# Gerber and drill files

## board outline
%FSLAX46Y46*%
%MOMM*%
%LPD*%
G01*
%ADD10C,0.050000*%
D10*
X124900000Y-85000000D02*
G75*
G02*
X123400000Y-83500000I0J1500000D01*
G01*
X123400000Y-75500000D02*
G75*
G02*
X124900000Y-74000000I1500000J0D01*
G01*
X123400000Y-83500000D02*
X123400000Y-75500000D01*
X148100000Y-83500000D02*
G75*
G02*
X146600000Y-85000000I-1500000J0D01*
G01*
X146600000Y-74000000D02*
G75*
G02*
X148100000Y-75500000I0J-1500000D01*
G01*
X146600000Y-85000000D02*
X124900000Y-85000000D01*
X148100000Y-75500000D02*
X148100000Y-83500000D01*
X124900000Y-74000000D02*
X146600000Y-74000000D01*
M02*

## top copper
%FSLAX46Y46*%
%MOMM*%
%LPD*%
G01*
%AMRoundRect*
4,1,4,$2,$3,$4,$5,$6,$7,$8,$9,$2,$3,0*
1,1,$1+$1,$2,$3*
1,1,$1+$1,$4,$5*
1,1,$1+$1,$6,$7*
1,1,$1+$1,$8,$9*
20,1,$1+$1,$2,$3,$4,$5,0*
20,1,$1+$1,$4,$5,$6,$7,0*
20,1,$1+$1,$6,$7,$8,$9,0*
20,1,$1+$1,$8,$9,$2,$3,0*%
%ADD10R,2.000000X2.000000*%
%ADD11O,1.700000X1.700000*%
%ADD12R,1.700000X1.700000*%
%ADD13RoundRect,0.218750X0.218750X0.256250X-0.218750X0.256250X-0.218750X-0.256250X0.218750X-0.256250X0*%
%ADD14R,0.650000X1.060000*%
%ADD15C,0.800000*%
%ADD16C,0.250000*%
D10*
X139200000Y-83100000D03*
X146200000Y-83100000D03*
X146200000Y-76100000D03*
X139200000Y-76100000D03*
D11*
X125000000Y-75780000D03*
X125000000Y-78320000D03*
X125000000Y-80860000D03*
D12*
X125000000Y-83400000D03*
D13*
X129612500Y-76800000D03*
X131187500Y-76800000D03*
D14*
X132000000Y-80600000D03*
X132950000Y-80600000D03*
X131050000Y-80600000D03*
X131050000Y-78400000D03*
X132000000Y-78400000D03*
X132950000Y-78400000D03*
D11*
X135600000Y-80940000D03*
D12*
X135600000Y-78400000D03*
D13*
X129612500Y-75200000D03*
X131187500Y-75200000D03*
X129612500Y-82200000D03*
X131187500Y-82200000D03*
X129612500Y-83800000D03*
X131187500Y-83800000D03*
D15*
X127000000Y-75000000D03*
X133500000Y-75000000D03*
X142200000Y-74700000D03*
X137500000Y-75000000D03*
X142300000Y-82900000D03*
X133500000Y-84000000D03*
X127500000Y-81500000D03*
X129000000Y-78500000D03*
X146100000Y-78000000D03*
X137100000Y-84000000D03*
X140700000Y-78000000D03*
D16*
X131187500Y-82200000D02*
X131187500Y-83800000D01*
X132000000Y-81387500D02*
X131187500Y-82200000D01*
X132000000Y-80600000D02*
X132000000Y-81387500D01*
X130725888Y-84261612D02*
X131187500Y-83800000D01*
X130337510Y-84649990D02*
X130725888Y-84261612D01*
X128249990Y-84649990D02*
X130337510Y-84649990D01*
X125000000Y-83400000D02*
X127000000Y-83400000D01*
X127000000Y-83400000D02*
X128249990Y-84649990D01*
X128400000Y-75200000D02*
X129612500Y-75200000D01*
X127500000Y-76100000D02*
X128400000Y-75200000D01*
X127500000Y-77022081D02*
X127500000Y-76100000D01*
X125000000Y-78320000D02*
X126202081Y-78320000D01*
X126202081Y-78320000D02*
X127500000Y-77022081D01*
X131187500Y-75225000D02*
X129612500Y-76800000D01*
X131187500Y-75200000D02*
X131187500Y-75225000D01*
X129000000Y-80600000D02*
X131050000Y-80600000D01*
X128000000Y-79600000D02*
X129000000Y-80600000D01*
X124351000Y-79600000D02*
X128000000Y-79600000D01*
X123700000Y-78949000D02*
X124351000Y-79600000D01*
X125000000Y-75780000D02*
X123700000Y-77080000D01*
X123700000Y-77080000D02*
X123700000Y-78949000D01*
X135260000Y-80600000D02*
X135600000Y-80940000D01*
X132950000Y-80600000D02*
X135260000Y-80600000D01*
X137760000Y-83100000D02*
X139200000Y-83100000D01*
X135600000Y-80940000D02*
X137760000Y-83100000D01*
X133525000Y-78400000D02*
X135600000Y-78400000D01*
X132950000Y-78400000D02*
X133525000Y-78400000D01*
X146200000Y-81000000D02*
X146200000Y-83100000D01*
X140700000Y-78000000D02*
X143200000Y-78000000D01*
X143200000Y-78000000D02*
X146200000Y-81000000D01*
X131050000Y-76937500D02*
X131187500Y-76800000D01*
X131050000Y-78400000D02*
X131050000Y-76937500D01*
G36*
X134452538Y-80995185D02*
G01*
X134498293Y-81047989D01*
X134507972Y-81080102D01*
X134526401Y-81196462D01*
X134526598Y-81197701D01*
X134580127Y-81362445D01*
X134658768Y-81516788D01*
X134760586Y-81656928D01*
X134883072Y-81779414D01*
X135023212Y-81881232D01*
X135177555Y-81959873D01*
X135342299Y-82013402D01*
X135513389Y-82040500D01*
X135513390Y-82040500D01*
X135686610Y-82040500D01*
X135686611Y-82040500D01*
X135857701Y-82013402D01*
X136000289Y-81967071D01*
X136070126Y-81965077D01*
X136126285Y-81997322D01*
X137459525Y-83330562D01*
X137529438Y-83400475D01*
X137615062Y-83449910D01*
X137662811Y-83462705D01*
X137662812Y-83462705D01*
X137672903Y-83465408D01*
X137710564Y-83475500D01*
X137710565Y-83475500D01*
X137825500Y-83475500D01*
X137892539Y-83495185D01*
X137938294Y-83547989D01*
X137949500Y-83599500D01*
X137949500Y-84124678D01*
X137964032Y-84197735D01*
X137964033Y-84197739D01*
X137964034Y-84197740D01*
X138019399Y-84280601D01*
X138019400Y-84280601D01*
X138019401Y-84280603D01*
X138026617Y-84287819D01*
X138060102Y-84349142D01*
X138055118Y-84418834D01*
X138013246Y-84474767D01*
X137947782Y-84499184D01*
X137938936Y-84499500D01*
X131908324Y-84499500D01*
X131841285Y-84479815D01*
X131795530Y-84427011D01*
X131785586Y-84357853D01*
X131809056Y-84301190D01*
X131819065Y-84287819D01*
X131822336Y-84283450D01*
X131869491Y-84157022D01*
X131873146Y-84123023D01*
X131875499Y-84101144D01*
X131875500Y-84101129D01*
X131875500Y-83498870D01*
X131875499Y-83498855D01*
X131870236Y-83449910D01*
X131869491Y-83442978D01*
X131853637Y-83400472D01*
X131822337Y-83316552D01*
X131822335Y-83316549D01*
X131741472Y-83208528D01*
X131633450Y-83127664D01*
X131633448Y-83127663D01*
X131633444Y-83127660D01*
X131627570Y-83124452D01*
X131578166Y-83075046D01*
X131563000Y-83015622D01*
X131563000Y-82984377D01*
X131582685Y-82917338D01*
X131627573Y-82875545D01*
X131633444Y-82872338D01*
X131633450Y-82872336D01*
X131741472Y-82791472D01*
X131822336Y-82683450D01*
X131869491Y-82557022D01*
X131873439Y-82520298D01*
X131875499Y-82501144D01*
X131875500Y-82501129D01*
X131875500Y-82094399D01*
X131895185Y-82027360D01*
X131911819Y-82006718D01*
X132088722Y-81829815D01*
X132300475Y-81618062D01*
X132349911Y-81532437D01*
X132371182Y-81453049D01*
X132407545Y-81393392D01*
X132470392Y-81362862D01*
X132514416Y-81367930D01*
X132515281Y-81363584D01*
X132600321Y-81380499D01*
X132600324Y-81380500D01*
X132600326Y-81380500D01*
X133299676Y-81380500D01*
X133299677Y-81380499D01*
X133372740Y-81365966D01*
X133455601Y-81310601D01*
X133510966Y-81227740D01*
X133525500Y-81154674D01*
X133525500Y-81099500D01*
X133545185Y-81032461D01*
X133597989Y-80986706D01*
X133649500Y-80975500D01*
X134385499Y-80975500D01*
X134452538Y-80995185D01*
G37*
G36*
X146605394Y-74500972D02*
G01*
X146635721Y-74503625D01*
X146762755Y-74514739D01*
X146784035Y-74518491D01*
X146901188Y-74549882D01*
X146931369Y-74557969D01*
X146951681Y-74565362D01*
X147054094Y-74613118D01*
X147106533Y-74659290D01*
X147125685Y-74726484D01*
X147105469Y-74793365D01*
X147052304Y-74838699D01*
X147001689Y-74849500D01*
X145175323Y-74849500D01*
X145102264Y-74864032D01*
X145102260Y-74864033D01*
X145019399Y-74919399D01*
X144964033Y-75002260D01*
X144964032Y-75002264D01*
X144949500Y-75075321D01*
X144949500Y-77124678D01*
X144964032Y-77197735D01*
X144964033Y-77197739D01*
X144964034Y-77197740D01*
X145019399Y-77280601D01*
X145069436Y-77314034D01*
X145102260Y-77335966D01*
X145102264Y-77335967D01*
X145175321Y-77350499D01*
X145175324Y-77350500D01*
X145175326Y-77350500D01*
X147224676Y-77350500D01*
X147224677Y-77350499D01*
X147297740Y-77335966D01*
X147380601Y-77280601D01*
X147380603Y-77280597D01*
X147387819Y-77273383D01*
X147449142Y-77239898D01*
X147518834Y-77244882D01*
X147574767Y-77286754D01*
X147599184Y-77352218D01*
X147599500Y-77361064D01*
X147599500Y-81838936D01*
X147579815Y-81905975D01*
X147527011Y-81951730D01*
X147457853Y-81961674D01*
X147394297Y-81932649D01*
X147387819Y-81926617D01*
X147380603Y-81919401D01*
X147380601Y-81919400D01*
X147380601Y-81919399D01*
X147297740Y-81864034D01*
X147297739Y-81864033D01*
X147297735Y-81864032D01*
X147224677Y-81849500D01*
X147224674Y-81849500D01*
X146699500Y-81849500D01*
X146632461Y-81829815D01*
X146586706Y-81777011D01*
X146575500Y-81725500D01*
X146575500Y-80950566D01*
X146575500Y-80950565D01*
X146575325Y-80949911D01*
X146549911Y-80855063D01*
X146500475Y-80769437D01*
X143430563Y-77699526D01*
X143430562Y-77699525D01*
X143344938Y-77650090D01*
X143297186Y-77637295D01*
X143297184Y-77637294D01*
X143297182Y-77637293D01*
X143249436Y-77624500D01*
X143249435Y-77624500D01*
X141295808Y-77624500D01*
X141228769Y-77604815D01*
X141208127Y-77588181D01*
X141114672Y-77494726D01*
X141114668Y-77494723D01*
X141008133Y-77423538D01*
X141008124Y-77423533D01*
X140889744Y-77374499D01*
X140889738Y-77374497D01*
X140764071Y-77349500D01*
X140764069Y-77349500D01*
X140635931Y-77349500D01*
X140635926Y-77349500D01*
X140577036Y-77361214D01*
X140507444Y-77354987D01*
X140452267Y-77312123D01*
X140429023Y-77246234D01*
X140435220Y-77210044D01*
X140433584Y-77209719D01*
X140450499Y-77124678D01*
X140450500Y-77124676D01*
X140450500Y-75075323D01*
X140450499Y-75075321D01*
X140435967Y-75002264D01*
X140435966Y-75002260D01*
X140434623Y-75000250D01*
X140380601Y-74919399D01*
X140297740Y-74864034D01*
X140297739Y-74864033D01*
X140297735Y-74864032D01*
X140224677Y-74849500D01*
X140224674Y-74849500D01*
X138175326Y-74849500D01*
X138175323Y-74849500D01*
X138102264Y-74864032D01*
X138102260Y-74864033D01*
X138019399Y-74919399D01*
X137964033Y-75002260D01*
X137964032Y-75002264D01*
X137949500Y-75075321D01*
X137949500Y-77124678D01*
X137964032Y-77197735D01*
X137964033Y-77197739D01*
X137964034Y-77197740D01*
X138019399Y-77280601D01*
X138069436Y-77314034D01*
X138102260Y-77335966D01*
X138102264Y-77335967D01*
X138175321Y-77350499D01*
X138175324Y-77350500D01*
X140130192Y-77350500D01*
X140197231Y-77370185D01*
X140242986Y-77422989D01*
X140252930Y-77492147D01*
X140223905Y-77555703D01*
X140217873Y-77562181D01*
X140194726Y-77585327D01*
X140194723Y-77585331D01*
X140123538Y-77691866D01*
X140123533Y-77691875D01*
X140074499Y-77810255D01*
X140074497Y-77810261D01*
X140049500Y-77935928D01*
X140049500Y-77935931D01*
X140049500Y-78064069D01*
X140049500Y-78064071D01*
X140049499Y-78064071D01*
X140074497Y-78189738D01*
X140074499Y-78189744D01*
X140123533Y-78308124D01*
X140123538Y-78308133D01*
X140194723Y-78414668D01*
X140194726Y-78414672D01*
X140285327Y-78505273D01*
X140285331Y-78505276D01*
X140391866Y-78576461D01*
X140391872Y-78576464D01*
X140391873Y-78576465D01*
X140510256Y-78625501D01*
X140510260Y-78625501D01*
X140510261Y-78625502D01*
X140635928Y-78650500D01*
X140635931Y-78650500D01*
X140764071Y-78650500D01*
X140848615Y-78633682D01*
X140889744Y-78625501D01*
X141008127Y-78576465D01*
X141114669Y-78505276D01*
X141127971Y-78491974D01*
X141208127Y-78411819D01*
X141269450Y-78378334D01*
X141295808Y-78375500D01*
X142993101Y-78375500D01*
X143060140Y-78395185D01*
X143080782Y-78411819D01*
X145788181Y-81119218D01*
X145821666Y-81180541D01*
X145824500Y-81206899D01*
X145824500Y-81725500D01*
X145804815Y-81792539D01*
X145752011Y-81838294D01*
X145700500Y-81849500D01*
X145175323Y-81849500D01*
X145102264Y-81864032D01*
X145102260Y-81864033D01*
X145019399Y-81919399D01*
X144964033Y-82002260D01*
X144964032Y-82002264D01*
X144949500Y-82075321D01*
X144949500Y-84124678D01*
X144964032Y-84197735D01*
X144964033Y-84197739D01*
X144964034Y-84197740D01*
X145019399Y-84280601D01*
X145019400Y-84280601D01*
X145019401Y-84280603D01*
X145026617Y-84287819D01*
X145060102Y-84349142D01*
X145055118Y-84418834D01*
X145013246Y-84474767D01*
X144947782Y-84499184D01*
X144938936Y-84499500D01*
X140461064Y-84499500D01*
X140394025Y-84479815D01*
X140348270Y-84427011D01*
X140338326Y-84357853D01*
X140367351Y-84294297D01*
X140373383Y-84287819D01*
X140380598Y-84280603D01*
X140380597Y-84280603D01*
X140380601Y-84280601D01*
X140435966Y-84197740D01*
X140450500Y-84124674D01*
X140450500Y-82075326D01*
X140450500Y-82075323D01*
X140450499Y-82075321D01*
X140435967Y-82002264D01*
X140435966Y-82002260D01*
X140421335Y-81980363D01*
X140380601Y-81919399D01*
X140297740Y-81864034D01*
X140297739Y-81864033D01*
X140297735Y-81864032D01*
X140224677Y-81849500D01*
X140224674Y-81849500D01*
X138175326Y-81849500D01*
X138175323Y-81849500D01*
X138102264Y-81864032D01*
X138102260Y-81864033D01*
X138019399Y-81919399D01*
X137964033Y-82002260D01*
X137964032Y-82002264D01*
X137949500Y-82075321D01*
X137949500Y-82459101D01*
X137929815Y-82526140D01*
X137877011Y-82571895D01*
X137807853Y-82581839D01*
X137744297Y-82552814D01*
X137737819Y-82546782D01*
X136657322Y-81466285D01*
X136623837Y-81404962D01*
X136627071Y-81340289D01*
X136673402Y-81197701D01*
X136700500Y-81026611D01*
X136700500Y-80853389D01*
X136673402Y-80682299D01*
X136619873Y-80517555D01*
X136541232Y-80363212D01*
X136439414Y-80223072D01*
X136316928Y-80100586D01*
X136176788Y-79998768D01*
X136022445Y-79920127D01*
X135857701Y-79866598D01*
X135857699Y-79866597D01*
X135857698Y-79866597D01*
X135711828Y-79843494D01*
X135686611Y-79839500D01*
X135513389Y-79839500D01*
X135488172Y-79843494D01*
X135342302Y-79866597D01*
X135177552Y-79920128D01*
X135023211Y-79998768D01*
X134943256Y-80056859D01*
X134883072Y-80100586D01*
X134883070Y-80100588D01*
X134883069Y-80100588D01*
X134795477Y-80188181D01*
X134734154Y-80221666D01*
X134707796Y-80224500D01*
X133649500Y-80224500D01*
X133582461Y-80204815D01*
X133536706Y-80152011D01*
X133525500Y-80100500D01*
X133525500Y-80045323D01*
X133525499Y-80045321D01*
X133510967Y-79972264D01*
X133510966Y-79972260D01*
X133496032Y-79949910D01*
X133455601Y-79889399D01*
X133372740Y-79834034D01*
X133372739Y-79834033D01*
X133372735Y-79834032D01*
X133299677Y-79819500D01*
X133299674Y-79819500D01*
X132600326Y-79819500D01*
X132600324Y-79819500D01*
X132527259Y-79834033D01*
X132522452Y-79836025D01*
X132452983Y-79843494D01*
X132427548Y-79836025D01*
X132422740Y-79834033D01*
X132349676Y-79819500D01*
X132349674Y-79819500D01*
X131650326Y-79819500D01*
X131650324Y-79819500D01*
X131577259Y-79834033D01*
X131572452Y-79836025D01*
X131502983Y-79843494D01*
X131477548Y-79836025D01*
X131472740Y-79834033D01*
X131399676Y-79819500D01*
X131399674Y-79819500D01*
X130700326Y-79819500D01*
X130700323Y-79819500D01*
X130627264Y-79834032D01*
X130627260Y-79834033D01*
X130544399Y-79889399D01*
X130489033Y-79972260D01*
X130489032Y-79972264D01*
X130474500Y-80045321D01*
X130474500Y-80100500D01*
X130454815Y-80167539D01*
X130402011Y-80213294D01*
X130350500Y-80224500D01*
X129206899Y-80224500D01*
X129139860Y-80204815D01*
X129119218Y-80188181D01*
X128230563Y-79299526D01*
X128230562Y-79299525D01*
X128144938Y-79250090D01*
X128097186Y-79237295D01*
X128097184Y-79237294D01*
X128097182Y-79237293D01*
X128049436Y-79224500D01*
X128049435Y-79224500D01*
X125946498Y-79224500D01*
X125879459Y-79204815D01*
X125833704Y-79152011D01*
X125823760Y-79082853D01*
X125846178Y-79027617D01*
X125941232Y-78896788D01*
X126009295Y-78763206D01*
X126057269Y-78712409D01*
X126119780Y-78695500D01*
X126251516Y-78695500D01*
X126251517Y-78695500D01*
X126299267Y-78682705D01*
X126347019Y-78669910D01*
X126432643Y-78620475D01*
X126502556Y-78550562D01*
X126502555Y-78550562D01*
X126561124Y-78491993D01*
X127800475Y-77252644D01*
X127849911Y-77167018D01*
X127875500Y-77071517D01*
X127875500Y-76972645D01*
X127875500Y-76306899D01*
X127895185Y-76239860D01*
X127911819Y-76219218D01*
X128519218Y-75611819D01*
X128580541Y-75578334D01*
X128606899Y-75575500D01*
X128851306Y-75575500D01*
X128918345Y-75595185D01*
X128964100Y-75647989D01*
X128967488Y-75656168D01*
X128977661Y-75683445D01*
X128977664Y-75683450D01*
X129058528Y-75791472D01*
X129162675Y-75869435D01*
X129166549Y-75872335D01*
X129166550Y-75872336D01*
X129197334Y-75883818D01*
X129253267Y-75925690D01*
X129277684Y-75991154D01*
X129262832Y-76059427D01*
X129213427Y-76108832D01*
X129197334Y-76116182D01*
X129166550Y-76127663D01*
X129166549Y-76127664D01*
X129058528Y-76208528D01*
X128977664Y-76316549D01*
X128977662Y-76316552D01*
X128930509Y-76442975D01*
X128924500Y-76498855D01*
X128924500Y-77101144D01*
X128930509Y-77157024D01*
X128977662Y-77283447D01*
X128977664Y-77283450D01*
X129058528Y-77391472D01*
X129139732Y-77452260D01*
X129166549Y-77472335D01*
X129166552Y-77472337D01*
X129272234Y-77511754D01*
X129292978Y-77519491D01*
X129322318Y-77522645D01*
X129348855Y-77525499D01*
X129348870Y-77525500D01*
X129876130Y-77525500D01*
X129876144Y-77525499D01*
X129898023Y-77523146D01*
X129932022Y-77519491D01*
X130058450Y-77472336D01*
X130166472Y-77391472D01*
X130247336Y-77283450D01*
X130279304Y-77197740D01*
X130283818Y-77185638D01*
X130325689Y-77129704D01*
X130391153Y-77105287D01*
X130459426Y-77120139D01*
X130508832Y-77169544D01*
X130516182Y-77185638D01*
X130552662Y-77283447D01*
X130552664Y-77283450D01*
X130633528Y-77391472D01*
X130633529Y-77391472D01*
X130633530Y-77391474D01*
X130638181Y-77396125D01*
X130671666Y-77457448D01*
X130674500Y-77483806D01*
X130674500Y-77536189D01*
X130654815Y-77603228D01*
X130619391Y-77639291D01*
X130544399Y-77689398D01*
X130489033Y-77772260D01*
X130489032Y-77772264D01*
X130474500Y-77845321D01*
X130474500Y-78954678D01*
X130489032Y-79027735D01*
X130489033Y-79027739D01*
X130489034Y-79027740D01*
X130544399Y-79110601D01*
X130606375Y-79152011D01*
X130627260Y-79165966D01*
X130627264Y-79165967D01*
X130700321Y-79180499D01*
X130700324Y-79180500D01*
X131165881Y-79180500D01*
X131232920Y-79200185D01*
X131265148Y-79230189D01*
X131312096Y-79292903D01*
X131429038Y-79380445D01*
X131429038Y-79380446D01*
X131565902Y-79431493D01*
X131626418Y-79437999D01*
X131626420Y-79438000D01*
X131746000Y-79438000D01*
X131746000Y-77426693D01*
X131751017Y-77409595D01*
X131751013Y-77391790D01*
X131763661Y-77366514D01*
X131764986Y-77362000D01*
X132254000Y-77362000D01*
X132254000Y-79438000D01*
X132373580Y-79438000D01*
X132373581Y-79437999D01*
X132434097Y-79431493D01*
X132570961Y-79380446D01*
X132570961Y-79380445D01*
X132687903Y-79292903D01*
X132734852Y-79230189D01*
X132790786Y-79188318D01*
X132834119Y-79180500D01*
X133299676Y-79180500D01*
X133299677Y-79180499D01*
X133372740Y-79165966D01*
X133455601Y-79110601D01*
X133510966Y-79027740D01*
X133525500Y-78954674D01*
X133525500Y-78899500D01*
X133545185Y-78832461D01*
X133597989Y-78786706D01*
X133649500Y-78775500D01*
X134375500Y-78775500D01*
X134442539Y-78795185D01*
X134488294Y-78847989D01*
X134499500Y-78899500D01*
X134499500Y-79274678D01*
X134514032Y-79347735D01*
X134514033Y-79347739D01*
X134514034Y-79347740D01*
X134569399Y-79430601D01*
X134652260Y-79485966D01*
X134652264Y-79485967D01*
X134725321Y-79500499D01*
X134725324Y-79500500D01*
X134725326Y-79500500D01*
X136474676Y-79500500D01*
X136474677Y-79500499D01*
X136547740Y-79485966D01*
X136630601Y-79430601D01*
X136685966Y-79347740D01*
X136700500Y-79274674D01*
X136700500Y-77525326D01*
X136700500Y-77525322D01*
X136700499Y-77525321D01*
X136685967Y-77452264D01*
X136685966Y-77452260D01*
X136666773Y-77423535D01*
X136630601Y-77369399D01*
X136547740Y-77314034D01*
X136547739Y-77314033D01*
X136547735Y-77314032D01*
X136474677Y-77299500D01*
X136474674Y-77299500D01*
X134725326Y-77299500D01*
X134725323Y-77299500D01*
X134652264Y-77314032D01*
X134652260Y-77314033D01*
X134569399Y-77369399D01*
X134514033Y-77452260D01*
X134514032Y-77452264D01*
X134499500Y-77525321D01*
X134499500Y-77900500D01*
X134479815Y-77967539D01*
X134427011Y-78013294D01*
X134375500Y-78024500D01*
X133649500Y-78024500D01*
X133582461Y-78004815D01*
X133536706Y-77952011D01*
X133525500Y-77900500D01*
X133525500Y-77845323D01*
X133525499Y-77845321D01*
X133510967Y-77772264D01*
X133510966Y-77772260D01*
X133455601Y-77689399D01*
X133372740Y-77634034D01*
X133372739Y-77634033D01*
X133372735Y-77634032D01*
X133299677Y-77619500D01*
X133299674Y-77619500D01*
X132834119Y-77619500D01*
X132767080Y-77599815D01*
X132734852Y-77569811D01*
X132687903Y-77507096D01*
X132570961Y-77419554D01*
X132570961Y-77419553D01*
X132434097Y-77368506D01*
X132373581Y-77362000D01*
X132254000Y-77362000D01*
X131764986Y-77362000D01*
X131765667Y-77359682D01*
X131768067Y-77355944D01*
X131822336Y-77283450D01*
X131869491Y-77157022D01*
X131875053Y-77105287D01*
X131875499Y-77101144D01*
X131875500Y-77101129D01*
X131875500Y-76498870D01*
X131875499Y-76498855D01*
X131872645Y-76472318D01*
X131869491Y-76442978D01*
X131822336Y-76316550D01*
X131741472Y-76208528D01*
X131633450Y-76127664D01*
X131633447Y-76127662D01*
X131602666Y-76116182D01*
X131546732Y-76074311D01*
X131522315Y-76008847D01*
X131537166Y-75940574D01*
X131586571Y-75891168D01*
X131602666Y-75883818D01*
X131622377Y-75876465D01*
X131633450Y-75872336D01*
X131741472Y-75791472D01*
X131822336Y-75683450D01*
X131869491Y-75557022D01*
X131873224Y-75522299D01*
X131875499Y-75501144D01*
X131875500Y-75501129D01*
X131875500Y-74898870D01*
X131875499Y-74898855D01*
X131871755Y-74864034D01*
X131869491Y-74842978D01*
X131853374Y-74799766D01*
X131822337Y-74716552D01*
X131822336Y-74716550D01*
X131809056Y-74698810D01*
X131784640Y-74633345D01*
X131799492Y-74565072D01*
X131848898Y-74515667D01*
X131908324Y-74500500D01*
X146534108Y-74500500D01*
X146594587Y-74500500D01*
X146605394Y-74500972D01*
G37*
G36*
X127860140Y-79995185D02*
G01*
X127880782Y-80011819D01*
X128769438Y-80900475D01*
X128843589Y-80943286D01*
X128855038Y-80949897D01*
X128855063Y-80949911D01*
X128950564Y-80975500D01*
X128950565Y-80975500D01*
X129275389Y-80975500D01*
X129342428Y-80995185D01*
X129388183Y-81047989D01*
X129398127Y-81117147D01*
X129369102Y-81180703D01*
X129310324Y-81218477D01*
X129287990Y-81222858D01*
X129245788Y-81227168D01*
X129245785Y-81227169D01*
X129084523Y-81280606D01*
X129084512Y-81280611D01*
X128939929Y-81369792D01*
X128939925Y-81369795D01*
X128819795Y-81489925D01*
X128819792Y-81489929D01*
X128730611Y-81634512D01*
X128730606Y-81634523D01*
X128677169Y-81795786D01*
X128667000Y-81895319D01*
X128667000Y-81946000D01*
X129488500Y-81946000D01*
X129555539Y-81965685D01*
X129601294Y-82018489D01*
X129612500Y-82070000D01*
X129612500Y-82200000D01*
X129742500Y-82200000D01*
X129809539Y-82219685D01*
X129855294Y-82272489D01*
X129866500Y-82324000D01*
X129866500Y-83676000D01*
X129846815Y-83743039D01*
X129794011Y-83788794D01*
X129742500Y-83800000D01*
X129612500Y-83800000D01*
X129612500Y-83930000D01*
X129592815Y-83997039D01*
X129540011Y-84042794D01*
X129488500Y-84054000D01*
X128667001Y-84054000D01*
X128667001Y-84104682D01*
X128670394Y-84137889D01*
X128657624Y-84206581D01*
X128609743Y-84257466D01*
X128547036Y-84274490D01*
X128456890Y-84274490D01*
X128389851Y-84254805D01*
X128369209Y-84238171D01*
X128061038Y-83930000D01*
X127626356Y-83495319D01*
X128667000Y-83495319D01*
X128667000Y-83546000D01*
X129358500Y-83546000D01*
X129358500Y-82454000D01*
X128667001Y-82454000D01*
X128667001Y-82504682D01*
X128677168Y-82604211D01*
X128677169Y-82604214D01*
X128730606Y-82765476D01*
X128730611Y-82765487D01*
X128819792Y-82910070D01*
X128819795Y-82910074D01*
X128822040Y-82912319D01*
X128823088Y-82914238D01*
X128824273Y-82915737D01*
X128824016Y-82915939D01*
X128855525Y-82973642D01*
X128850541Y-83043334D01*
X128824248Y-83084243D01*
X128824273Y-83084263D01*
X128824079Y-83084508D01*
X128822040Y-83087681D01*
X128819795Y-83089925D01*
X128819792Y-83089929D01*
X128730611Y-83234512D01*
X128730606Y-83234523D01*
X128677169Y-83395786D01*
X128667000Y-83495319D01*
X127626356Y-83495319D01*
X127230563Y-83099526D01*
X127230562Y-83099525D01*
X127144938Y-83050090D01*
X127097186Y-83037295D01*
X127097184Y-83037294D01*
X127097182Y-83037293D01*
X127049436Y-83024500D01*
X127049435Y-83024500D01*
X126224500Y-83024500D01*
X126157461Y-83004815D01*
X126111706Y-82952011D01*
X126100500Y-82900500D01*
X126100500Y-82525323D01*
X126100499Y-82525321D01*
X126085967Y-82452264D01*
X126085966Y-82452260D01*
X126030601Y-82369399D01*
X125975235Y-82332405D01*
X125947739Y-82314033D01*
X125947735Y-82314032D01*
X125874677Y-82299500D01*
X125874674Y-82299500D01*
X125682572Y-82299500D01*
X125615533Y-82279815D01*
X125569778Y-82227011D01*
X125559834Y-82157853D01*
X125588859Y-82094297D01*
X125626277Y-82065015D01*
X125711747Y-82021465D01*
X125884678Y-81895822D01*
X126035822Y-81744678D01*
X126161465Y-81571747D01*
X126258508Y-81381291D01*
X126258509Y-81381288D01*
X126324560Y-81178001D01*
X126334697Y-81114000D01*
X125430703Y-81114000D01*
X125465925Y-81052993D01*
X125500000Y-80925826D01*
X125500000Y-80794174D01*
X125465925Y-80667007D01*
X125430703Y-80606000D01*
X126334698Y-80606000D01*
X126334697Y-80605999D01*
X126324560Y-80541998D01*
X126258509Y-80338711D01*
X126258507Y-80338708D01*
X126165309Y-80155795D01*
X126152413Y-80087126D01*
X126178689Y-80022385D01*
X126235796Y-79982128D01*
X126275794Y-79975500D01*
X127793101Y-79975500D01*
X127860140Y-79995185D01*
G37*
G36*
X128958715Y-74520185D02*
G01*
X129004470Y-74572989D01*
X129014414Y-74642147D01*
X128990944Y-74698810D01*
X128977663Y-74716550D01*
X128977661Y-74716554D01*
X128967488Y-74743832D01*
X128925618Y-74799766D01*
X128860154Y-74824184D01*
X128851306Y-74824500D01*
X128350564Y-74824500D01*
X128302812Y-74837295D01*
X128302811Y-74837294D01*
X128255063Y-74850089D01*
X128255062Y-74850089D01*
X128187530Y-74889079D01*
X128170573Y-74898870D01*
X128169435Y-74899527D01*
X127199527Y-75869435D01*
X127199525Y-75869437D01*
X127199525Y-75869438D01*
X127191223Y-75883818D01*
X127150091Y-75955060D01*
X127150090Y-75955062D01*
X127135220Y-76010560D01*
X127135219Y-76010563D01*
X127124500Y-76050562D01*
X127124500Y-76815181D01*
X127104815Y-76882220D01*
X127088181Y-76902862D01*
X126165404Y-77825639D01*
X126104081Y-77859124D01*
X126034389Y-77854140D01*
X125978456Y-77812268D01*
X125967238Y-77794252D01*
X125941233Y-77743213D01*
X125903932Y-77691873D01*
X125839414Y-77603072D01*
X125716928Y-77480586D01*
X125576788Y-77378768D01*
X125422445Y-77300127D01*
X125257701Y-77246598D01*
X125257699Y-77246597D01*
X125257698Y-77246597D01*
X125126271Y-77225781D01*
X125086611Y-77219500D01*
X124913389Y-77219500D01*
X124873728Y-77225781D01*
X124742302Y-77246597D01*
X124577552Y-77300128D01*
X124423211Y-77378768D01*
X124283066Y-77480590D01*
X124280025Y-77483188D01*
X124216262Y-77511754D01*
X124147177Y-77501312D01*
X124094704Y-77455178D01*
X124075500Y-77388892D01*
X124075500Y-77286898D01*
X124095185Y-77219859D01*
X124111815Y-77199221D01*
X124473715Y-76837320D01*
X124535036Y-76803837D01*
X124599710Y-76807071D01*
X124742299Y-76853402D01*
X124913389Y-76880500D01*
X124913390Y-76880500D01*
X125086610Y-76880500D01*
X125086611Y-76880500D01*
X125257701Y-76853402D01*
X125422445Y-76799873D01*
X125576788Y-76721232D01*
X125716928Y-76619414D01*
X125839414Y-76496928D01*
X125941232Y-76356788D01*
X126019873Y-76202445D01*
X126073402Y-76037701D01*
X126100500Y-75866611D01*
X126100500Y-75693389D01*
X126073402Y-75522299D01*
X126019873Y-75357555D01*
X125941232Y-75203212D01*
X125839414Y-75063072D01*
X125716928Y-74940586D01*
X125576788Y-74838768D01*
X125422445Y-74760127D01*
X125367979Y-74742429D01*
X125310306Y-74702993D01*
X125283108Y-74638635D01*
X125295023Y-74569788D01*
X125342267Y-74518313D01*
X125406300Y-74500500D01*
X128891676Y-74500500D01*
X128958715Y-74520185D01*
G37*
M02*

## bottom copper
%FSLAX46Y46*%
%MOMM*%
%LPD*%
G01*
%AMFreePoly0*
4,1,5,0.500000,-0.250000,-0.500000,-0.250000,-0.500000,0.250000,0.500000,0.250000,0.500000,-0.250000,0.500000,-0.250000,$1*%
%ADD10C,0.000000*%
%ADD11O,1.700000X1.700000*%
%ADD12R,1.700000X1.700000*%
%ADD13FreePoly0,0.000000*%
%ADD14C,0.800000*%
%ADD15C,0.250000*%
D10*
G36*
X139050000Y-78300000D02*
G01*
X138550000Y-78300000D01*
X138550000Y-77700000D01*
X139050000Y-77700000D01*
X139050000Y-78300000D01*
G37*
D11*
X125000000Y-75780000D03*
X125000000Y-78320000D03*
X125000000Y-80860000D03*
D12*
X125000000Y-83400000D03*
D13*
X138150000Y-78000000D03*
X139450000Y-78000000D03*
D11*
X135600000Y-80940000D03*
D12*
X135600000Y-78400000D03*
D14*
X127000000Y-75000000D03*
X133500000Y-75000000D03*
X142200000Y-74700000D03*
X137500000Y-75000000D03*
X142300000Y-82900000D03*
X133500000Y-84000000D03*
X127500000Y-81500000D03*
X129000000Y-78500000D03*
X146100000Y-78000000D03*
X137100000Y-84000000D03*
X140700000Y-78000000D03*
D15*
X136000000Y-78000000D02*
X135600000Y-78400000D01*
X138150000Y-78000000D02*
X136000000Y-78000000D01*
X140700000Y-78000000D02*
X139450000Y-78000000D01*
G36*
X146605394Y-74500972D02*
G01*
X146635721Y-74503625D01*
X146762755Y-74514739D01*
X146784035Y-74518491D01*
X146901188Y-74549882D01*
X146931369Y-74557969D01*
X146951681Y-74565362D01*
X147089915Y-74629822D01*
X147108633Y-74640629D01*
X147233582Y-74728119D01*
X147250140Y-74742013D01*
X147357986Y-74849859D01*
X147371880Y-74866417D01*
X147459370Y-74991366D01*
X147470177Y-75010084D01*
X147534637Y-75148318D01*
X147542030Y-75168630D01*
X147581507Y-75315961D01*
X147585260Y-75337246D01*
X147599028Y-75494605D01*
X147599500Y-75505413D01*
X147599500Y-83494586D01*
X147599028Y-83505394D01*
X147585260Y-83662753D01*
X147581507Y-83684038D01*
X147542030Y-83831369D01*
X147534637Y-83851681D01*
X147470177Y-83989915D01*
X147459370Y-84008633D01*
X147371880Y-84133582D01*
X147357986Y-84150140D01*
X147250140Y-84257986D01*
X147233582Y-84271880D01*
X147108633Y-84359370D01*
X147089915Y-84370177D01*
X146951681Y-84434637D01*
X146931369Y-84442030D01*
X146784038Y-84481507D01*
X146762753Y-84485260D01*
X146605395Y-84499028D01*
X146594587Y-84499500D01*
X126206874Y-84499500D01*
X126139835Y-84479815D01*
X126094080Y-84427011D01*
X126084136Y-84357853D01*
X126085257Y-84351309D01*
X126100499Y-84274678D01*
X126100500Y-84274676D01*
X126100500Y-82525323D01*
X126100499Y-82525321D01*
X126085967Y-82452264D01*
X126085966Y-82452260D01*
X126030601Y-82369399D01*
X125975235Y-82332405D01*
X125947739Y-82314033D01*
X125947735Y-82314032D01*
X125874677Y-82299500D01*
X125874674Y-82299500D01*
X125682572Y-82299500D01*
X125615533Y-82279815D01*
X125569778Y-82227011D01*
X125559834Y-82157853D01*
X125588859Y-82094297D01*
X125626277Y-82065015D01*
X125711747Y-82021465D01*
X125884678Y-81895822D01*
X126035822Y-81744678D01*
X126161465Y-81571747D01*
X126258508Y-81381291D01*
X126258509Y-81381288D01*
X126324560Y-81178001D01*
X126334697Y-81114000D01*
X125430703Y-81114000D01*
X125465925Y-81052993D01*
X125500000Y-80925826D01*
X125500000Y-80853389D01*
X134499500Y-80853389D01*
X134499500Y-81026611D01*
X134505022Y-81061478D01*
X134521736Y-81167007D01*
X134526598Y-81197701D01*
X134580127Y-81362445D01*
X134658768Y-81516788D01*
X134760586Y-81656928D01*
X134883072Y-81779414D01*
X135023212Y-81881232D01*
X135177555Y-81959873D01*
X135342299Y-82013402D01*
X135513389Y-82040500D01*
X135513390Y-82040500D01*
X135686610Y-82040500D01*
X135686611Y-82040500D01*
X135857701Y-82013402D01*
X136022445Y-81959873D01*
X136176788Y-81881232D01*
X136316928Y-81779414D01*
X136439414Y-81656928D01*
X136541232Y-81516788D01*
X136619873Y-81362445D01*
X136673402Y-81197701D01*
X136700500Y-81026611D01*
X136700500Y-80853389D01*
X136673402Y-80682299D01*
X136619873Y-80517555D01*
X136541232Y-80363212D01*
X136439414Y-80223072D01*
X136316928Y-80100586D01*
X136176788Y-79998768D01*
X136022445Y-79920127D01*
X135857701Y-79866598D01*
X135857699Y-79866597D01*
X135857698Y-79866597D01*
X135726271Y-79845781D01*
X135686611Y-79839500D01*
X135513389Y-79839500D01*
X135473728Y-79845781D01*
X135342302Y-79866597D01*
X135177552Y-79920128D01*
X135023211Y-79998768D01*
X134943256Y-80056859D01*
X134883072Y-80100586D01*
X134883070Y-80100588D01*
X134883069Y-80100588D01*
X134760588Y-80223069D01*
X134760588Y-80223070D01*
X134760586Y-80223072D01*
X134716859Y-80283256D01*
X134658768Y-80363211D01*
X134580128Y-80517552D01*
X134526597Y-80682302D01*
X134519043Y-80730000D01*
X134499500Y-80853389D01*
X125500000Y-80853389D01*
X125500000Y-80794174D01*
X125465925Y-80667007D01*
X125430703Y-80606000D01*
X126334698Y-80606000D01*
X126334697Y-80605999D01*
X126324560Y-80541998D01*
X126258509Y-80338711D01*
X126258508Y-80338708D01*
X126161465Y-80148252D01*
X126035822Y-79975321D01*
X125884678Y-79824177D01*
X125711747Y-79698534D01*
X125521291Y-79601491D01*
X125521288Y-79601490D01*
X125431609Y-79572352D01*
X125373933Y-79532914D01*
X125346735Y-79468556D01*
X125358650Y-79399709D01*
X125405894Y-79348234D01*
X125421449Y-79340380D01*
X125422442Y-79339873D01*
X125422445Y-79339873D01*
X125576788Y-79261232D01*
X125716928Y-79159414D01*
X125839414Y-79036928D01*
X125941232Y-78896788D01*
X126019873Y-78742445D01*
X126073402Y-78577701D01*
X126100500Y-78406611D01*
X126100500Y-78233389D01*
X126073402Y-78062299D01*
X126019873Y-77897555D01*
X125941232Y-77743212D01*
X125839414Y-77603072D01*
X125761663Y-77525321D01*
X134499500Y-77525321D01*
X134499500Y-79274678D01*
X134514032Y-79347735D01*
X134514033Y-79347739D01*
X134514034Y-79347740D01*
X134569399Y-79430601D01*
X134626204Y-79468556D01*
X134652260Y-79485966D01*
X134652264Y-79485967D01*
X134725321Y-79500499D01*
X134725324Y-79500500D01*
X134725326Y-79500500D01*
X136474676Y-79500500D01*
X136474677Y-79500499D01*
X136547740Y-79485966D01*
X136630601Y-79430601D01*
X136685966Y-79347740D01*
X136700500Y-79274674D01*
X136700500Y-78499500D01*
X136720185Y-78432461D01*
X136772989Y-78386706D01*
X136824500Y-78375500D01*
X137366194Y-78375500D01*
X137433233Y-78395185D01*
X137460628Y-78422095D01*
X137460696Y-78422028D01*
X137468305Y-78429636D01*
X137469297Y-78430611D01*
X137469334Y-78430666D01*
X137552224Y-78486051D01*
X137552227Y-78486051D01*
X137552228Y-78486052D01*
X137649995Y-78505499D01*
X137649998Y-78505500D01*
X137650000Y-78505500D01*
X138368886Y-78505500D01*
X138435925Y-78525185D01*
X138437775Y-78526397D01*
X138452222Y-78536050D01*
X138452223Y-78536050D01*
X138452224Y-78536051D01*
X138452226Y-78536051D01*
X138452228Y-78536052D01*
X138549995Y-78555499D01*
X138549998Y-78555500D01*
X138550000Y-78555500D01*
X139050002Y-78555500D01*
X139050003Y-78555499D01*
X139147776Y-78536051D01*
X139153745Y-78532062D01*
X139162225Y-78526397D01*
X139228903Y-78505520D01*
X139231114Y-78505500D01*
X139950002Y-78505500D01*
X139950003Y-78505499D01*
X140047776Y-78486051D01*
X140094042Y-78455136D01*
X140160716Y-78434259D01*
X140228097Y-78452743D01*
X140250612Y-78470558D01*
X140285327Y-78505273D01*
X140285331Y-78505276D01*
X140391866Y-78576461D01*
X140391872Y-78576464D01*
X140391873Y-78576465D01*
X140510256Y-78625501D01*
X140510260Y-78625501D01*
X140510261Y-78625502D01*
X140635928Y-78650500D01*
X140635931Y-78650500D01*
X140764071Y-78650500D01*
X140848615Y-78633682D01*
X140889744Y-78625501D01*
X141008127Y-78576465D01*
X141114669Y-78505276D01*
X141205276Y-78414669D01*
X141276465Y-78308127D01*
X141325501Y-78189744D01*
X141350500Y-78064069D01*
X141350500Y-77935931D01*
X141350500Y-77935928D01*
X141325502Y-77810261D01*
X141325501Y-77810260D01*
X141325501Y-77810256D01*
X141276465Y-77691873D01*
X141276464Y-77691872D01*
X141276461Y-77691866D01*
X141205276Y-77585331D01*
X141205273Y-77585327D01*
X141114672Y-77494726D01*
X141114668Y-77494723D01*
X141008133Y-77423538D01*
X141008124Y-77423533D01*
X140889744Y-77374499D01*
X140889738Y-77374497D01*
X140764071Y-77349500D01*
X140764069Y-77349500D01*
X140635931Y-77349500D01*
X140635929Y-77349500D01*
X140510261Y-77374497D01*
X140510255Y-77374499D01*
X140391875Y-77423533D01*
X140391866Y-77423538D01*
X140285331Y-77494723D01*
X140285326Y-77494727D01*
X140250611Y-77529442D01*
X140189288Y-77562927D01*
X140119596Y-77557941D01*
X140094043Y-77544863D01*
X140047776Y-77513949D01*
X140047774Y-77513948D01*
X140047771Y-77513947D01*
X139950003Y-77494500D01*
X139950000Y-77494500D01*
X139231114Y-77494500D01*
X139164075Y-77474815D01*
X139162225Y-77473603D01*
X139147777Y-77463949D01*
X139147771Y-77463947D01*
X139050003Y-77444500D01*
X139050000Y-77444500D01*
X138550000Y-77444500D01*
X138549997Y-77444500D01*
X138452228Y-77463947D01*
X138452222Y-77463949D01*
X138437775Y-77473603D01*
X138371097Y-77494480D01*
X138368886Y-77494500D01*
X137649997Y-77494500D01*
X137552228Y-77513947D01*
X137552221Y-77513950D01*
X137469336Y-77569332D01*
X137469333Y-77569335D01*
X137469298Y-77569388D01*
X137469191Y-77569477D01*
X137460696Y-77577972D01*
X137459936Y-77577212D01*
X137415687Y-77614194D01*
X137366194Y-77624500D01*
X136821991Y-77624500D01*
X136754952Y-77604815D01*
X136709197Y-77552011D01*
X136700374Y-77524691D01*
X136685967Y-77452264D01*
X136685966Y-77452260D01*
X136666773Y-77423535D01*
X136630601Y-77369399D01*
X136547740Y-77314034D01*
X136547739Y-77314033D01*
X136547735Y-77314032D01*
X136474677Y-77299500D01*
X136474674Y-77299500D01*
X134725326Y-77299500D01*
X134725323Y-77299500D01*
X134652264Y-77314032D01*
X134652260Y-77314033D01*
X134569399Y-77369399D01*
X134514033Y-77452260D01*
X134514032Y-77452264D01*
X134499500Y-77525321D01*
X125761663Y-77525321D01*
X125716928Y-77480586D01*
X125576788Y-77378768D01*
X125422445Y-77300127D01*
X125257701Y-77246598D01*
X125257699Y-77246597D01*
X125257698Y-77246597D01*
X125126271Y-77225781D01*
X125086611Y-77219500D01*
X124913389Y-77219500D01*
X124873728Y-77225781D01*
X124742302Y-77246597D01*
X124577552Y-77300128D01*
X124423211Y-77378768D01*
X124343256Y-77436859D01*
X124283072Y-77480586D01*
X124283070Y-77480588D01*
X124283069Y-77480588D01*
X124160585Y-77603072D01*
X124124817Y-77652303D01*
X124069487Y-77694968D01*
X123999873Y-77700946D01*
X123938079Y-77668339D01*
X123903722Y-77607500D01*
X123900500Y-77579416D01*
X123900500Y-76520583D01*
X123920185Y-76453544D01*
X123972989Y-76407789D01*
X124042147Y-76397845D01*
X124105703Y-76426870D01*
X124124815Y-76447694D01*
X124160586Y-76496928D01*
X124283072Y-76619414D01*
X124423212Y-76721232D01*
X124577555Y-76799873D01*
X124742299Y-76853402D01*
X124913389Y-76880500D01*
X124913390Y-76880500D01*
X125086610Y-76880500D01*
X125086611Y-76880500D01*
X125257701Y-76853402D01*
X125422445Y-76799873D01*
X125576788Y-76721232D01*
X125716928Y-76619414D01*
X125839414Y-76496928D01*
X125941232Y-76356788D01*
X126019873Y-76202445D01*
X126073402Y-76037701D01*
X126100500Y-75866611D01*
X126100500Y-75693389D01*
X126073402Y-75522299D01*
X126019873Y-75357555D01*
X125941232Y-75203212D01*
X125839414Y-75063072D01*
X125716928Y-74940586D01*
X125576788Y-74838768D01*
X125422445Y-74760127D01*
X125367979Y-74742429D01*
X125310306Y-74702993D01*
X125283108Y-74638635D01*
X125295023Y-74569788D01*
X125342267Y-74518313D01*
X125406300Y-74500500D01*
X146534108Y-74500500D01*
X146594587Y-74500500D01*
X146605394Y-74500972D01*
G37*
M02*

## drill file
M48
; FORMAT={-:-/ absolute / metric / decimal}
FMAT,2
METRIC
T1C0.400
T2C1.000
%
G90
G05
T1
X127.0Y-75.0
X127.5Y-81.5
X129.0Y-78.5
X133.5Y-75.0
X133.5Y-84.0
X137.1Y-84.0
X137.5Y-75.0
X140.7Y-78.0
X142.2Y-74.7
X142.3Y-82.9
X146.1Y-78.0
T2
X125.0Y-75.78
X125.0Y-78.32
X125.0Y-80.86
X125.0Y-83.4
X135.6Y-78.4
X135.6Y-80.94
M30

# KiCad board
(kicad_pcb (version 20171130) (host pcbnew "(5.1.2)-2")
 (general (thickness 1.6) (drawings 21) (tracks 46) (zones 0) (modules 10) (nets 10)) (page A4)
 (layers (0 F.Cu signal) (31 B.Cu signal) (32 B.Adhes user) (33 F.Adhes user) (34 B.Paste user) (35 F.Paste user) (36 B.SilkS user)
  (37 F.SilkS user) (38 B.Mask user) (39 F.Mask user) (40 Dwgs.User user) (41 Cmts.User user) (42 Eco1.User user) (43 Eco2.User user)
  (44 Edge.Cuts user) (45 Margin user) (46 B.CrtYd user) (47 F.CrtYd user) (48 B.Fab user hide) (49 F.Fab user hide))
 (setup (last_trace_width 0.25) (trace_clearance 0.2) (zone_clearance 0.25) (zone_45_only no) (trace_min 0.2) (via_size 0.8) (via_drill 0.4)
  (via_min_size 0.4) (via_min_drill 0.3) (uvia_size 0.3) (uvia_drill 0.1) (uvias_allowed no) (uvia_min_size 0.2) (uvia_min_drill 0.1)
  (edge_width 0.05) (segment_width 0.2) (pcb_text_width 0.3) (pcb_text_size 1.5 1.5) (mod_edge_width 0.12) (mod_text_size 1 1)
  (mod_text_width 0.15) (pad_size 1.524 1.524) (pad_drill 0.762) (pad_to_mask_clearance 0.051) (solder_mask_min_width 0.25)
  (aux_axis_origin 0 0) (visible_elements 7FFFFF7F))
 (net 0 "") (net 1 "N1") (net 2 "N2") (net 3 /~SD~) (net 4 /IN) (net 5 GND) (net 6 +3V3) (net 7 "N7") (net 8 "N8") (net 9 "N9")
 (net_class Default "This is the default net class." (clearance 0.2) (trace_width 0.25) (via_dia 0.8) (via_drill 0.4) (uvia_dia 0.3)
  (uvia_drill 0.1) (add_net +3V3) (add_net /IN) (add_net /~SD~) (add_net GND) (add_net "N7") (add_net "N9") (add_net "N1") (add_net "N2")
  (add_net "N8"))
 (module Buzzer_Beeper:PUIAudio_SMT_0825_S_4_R (layer F.Cu) (at 142.7 79.6 90)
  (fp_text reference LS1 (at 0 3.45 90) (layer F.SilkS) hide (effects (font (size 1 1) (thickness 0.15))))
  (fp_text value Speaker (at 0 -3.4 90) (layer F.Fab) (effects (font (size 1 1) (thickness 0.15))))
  (pad 1 smd rect (at -3.5 -3.5) (size 2 2) (layers F.Cu F.Paste F.Mask) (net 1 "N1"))
  (pad 2 smd rect (at -3.5 3.5) (size 2 2) (layers F.Cu F.Paste F.Mask) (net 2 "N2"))
  (pad 3 smd rect (at 3.5 3.5) (size 2 2) (layers F.Cu F.Paste F.Mask))
  (pad 4 smd rect (at 3.5 -3.5) (size 2 2) (layers F.Cu F.Paste F.Mask)))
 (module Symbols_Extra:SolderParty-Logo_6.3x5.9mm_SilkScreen (layer B.Cu) (at 129.8 81.5 180)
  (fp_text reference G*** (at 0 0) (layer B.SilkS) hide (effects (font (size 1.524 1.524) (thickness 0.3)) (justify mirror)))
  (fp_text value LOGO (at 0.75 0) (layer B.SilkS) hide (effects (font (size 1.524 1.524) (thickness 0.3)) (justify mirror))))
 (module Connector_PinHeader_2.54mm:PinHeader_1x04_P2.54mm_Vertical (layer F.Cu) (at 125 83.4 180)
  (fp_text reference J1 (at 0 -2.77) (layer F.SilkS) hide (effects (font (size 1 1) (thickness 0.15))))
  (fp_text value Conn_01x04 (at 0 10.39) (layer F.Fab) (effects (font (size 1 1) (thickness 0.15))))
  (pad 4 thru_hole oval (at 0 7.62 180) (size 1.7 1.7) (drill 1) (layers *.Cu *.Mask) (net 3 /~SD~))
  (pad 3 thru_hole oval (at 0 5.08 180) (size 1.7 1.7) (drill 1) (layers *.Cu *.Mask) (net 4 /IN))
  (pad 2 thru_hole oval (at 0 2.54 180) (size 1.7 1.7) (drill 1) (layers *.Cu *.Mask) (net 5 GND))
  (pad 1 thru_hole rect (at 0 0 180) (size 1.7 1.7) (drill 1) (layers *.Cu *.Mask) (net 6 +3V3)))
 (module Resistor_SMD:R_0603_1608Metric (layer F.Cu) (at 130.4 76.8 180)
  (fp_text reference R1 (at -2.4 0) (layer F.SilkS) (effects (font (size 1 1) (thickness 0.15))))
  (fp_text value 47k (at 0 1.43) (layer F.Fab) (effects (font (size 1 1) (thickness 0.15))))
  (pad 2 smd roundrect (at 0.7875 0 180) (size 0.875 0.95) (layers F.Cu F.Paste F.Mask) (roundrect_rratio 0.25) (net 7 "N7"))
  (pad 1 smd roundrect (at -0.7875 0 180) (size 0.875 0.95) (layers F.Cu F.Paste F.Mask) (roundrect_rratio 0.25) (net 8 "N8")))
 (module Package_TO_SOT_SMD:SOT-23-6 (layer F.Cu) (at 132 79.5 270)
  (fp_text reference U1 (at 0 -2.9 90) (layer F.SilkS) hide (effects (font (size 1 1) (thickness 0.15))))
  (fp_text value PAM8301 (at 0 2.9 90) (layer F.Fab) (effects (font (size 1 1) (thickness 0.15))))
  (pad 5 smd rect (at 1.1 0 270) (size 1.06 0.65) (layers F.Cu F.Paste F.Mask) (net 6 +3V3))
  (pad 6 smd rect (at 1.1 -0.95 270) (size 1.06 0.65) (layers F.Cu F.Paste F.Mask) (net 1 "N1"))
  (pad 4 smd rect (at 1.1 0.95 270) (size 1.06 0.65) (layers F.Cu F.Paste F.Mask) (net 3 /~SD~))
  (pad 3 smd rect (at -1.1 0.95 270) (size 1.06 0.65) (layers F.Cu F.Paste F.Mask) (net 8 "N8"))
  (pad 2 smd rect (at -1.1 0 270) (size 1.06 0.65) (layers F.Cu F.Paste F.Mask) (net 5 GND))
  (pad 1 smd rect (at -1.1 -0.95 270) (size 1.06 0.65) (layers F.Cu F.Paste F.Mask) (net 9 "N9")))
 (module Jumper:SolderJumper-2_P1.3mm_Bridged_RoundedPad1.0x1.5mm (layer B.Cu) (at 138.8 78)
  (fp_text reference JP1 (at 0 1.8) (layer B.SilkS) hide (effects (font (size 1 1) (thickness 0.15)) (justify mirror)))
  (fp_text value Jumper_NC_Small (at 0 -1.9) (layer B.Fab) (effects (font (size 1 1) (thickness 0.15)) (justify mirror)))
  (fp_poly (pts (xy 0.25 0.3) (xy -0.25 0.3) (xy -0.25 -0.3) (xy 0.25 -0.3)) (layer B.Cu) (width 0))
  (pad 1 smd custom (at -0.65 0) (size 1 0.5) (layers B.Cu B.Mask) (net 9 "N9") (zone_connect 2) (options (clearance outline) (anchor rect))
   (primitives))
  (pad 2 smd custom (at 0.65 0) (size 1 0.5) (layers B.Cu B.Mask) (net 2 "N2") (zone_connect 2) (options (clearance outline) (anchor rect))
   (primitives)))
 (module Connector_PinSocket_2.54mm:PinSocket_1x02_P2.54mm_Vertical (layer F.Cu) (at 135.6 78.4)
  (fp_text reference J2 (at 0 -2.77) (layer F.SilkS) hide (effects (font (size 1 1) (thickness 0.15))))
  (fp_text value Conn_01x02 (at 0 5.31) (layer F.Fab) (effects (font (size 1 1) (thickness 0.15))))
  (pad 2 thru_hole oval (at 0 2.54) (size 1.7 1.7) (drill 1) (layers *.Cu *.Mask) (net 1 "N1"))
  (pad 1 thru_hole rect (at 0 0) (size 1.7 1.7) (drill 1) (layers *.Cu *.Mask) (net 9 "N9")))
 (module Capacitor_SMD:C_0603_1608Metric (layer F.Cu) (at 130.4 75.2 180)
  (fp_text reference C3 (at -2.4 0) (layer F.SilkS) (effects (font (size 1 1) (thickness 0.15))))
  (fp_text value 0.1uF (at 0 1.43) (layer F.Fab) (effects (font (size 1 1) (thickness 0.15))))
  (pad 2 smd roundrect (at 0.7875 0 180) (size 0.875 0.95) (layers F.Cu F.Paste F.Mask) (roundrect_rratio 0.25) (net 4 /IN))
  (pad 1 smd roundrect (at -0.7875 0 180) (size 0.875 0.95) (layers F.Cu F.Paste F.Mask) (roundrect_rratio 0.25) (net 7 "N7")))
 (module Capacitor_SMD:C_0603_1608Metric (layer F.Cu) (at 130.4 82.2 180)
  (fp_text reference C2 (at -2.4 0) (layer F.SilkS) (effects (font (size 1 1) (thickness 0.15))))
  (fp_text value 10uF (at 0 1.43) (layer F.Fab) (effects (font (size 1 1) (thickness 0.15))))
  (pad 2 smd roundrect (at 0.7875 0 180) (size 0.875 0.95) (layers F.Cu F.Paste F.Mask) (roundrect_rratio 0.25) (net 5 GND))
  (pad 1 smd roundrect (at -0.7875 0 180) (size 0.875 0.95) (layers F.Cu F.Paste F.Mask) (roundrect_rratio 0.25) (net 6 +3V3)))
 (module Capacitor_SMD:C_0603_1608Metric (layer F.Cu) (at 130.4 83.8 180)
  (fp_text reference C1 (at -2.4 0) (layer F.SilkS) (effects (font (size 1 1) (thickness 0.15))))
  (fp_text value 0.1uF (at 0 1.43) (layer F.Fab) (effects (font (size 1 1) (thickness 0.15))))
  (pad 2 smd roundrect (at 0.7875 0 180) (size 0.875 0.95) (layers F.Cu F.Paste F.Mask) (roundrect_rratio 0.25) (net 5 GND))
  (pad 1 smd roundrect (at -0.7875 0 180) (size 0.875 0.95) (layers F.Cu F.Paste F.Mask) (roundrect_rratio 0.25) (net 6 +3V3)))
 (gr_arc (start 124.9 83.5) (end 123.4 83.5) (angle -90) (layer Edge.Cuts) (width 0.05))
 (gr_arc (start 124.9 75.5) (end 124.9 74) (angle -90) (layer Edge.Cuts) (width 0.05))
 (gr_line (start 123.4 83.5) (end 123.4 75.5) (layer Edge.Cuts) (width 0.05))
 (gr_arc (start 146.6 83.5) (end 146.6 85) (angle -90) (layer Edge.Cuts) (width 0.05))
 (gr_arc (start 146.6 75.5) (end 148.1 75.5) (angle -90) (layer Edge.Cuts) (width 0.05))
 (gr_line (start 146.6 85) (end 124.9 85) (layer Edge.Cuts) (width 0.05))
 (gr_line (start 148.1 75.5) (end 148.1 83.5) (layer Edge.Cuts) (width 0.05))
 (gr_line (start 124.9 74) (end 146.6 74) (layer Edge.Cuts) (width 0.05))
 (via (at 127 75) (size 0.8) (drill 0.4) (layers F.Cu B.Cu) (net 5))
 (via (at 133.5 75) (size 0.8) (drill 0.4) (layers F.Cu B.Cu) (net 5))
 (via (at 142.2 74.7) (size 0.8) (drill 0.4) (layers F.Cu B.Cu) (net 5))
 (via (at 137.5 75) (size 0.8) (drill 0.4) (layers F.Cu B.Cu) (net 5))
 (via (at 142.3 82.9) (size 0.8) (drill 0.4) (layers F.Cu B.Cu) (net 5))
 (via (at 133.5 84) (size 0.8) (drill 0.4) (layers F.Cu B.Cu) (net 5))
 (via (at 127.5 81.5) (size 0.8) (drill 0.4) (layers F.Cu B.Cu) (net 5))
 (via (at 129 78.5) (size 0.8) (drill 0.4) (layers F.Cu B.Cu) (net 5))
 (via (at 146.1 78) (size 0.8) (drill 0.4) (layers F.Cu B.Cu) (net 5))
 (via (at 137.1 84) (size 0.8) (drill 0.4) (layers F.Cu B.Cu) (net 5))
 (segment (start 131.1875 82.2) (end 131.1875 83.8) (width 0.25) (layer F.Cu) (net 6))
 (segment (start 132 81.3875) (end 131.1875 82.2) (width 0.25) (layer F.Cu) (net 6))
 (segment (start 132 80.6) (end 132 81.3875) (width 0.25) (layer F.Cu) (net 6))
 (segment (start 130.725888 84.261612) (end 131.1875 83.8) (width 0.25) (layer F.Cu) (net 6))
 (segment (start 130.33751 84.64999) (end 130.725888 84.261612) (width 0.25) (layer F.Cu) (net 6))
 (segment (start 128.24999 84.64999) (end 130.33751 84.64999) (width 0.25) (layer F.Cu) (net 6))
 (segment (start 125 83.4) (end 127 83.4) (width 0.25) (layer F.Cu) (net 6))
 (segment (start 127 83.4) (end 128.24999 84.64999) (width 0.25) (layer F.Cu) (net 6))
 (segment (start 128.4 75.2) (end 129.6125 75.2) (width 0.25) (layer F.Cu) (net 4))
 (segment (start 127.5 76.1) (end 128.4 75.2) (width 0.25) (layer F.Cu) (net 4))
 (segment (start 127.5 77.022081) (end 127.5 76.1) (width 0.25) (layer F.Cu) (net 4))
 (segment (start 125 78.32) (end 126.202081 78.32) (width 0.25) (layer F.Cu) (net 4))
 (segment (start 126.202081 78.32) (end 127.5 77.022081) (width 0.25) (layer F.Cu) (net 4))
 (segment (start 131.1875 75.225) (end 129.6125 76.8) (width 0.25) (layer F.Cu) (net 7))
 (segment (start 131.1875 75.2) (end 131.1875 75.225) (width 0.25) (layer F.Cu) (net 7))
 (segment (start 129 80.6) (end 131.05 80.6) (width 0.25) (layer F.Cu) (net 3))
 (segment (start 128 79.6) (end 129 80.6) (width 0.25) (layer F.Cu) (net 3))
 (segment (start 124.351 79.6) (end 128 79.6) (width 0.25) (layer F.Cu) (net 3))
 (segment (start 123.7 78.949) (end 124.351 79.6) (width 0.25) (layer F.Cu) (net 3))
 (segment (start 125 75.78) (end 123.7 77.08) (width 0.25) (layer F.Cu) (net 3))
 (segment (start 123.7 77.08) (end 123.7 78.949) (width 0.25) (layer F.Cu) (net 3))
 (segment (start 135.26 80.6) (end 135.6 80.94) (width 0.25) (layer F.Cu) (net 1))
 (segment (start 132.95 80.6) (end 135.26 80.6) (width 0.25) (layer F.Cu) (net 1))
 (segment (start 137.76 83.1) (end 139.2 83.1) (width 0.25) (layer F.Cu) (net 1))
 (segment (start 135.6 80.94) (end 137.76 83.1) (width 0.25) (layer F.Cu) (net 1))
 (segment (start 133.525 78.4) (end 135.6 78.4) (width 0.25) (layer F.Cu) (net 9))
 (segment (start 132.95 78.4) (end 133.525 78.4) (width 0.25) (layer F.Cu) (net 9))
 (segment (start 136 78) (end 135.6 78.4) (width 0.25) (layer B.Cu) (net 9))
 (segment (start 138.15 78) (end 136 78) (width 0.25) (layer B.Cu) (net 9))
 (via (at 140.7 78) (size 0.8) (drill 0.4) (layers F.Cu B.Cu) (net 2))
 (segment (start 140.7 78) (end 139.45 78) (width 0.25) (layer B.Cu) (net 2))
 (segment (start 146.2 81) (end 146.2 83.1) (width 0.25) (layer F.Cu) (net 2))
 (segment (start 140.7 78) (end 143.2 78) (width 0.25) (layer F.Cu) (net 2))
 (segment (start 143.2 78) (end 146.2 81) (width 0.25) (layer F.Cu) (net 2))
 (segment (start 131.05 76.9375) (end 131.1875 76.8) (width 0.25) (layer F.Cu) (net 8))
 (segment (start 131.05 78.4) (end 131.05 76.9375) (width 0.25) (layer F.Cu) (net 8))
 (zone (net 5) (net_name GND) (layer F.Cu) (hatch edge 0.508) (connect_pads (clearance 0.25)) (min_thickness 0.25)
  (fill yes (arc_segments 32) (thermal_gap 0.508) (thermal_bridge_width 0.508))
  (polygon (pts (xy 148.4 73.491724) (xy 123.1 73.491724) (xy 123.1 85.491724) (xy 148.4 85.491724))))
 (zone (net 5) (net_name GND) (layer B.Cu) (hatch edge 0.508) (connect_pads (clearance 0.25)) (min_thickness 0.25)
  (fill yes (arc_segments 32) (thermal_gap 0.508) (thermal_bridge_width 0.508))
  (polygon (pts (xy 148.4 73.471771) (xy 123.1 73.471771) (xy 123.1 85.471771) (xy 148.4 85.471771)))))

